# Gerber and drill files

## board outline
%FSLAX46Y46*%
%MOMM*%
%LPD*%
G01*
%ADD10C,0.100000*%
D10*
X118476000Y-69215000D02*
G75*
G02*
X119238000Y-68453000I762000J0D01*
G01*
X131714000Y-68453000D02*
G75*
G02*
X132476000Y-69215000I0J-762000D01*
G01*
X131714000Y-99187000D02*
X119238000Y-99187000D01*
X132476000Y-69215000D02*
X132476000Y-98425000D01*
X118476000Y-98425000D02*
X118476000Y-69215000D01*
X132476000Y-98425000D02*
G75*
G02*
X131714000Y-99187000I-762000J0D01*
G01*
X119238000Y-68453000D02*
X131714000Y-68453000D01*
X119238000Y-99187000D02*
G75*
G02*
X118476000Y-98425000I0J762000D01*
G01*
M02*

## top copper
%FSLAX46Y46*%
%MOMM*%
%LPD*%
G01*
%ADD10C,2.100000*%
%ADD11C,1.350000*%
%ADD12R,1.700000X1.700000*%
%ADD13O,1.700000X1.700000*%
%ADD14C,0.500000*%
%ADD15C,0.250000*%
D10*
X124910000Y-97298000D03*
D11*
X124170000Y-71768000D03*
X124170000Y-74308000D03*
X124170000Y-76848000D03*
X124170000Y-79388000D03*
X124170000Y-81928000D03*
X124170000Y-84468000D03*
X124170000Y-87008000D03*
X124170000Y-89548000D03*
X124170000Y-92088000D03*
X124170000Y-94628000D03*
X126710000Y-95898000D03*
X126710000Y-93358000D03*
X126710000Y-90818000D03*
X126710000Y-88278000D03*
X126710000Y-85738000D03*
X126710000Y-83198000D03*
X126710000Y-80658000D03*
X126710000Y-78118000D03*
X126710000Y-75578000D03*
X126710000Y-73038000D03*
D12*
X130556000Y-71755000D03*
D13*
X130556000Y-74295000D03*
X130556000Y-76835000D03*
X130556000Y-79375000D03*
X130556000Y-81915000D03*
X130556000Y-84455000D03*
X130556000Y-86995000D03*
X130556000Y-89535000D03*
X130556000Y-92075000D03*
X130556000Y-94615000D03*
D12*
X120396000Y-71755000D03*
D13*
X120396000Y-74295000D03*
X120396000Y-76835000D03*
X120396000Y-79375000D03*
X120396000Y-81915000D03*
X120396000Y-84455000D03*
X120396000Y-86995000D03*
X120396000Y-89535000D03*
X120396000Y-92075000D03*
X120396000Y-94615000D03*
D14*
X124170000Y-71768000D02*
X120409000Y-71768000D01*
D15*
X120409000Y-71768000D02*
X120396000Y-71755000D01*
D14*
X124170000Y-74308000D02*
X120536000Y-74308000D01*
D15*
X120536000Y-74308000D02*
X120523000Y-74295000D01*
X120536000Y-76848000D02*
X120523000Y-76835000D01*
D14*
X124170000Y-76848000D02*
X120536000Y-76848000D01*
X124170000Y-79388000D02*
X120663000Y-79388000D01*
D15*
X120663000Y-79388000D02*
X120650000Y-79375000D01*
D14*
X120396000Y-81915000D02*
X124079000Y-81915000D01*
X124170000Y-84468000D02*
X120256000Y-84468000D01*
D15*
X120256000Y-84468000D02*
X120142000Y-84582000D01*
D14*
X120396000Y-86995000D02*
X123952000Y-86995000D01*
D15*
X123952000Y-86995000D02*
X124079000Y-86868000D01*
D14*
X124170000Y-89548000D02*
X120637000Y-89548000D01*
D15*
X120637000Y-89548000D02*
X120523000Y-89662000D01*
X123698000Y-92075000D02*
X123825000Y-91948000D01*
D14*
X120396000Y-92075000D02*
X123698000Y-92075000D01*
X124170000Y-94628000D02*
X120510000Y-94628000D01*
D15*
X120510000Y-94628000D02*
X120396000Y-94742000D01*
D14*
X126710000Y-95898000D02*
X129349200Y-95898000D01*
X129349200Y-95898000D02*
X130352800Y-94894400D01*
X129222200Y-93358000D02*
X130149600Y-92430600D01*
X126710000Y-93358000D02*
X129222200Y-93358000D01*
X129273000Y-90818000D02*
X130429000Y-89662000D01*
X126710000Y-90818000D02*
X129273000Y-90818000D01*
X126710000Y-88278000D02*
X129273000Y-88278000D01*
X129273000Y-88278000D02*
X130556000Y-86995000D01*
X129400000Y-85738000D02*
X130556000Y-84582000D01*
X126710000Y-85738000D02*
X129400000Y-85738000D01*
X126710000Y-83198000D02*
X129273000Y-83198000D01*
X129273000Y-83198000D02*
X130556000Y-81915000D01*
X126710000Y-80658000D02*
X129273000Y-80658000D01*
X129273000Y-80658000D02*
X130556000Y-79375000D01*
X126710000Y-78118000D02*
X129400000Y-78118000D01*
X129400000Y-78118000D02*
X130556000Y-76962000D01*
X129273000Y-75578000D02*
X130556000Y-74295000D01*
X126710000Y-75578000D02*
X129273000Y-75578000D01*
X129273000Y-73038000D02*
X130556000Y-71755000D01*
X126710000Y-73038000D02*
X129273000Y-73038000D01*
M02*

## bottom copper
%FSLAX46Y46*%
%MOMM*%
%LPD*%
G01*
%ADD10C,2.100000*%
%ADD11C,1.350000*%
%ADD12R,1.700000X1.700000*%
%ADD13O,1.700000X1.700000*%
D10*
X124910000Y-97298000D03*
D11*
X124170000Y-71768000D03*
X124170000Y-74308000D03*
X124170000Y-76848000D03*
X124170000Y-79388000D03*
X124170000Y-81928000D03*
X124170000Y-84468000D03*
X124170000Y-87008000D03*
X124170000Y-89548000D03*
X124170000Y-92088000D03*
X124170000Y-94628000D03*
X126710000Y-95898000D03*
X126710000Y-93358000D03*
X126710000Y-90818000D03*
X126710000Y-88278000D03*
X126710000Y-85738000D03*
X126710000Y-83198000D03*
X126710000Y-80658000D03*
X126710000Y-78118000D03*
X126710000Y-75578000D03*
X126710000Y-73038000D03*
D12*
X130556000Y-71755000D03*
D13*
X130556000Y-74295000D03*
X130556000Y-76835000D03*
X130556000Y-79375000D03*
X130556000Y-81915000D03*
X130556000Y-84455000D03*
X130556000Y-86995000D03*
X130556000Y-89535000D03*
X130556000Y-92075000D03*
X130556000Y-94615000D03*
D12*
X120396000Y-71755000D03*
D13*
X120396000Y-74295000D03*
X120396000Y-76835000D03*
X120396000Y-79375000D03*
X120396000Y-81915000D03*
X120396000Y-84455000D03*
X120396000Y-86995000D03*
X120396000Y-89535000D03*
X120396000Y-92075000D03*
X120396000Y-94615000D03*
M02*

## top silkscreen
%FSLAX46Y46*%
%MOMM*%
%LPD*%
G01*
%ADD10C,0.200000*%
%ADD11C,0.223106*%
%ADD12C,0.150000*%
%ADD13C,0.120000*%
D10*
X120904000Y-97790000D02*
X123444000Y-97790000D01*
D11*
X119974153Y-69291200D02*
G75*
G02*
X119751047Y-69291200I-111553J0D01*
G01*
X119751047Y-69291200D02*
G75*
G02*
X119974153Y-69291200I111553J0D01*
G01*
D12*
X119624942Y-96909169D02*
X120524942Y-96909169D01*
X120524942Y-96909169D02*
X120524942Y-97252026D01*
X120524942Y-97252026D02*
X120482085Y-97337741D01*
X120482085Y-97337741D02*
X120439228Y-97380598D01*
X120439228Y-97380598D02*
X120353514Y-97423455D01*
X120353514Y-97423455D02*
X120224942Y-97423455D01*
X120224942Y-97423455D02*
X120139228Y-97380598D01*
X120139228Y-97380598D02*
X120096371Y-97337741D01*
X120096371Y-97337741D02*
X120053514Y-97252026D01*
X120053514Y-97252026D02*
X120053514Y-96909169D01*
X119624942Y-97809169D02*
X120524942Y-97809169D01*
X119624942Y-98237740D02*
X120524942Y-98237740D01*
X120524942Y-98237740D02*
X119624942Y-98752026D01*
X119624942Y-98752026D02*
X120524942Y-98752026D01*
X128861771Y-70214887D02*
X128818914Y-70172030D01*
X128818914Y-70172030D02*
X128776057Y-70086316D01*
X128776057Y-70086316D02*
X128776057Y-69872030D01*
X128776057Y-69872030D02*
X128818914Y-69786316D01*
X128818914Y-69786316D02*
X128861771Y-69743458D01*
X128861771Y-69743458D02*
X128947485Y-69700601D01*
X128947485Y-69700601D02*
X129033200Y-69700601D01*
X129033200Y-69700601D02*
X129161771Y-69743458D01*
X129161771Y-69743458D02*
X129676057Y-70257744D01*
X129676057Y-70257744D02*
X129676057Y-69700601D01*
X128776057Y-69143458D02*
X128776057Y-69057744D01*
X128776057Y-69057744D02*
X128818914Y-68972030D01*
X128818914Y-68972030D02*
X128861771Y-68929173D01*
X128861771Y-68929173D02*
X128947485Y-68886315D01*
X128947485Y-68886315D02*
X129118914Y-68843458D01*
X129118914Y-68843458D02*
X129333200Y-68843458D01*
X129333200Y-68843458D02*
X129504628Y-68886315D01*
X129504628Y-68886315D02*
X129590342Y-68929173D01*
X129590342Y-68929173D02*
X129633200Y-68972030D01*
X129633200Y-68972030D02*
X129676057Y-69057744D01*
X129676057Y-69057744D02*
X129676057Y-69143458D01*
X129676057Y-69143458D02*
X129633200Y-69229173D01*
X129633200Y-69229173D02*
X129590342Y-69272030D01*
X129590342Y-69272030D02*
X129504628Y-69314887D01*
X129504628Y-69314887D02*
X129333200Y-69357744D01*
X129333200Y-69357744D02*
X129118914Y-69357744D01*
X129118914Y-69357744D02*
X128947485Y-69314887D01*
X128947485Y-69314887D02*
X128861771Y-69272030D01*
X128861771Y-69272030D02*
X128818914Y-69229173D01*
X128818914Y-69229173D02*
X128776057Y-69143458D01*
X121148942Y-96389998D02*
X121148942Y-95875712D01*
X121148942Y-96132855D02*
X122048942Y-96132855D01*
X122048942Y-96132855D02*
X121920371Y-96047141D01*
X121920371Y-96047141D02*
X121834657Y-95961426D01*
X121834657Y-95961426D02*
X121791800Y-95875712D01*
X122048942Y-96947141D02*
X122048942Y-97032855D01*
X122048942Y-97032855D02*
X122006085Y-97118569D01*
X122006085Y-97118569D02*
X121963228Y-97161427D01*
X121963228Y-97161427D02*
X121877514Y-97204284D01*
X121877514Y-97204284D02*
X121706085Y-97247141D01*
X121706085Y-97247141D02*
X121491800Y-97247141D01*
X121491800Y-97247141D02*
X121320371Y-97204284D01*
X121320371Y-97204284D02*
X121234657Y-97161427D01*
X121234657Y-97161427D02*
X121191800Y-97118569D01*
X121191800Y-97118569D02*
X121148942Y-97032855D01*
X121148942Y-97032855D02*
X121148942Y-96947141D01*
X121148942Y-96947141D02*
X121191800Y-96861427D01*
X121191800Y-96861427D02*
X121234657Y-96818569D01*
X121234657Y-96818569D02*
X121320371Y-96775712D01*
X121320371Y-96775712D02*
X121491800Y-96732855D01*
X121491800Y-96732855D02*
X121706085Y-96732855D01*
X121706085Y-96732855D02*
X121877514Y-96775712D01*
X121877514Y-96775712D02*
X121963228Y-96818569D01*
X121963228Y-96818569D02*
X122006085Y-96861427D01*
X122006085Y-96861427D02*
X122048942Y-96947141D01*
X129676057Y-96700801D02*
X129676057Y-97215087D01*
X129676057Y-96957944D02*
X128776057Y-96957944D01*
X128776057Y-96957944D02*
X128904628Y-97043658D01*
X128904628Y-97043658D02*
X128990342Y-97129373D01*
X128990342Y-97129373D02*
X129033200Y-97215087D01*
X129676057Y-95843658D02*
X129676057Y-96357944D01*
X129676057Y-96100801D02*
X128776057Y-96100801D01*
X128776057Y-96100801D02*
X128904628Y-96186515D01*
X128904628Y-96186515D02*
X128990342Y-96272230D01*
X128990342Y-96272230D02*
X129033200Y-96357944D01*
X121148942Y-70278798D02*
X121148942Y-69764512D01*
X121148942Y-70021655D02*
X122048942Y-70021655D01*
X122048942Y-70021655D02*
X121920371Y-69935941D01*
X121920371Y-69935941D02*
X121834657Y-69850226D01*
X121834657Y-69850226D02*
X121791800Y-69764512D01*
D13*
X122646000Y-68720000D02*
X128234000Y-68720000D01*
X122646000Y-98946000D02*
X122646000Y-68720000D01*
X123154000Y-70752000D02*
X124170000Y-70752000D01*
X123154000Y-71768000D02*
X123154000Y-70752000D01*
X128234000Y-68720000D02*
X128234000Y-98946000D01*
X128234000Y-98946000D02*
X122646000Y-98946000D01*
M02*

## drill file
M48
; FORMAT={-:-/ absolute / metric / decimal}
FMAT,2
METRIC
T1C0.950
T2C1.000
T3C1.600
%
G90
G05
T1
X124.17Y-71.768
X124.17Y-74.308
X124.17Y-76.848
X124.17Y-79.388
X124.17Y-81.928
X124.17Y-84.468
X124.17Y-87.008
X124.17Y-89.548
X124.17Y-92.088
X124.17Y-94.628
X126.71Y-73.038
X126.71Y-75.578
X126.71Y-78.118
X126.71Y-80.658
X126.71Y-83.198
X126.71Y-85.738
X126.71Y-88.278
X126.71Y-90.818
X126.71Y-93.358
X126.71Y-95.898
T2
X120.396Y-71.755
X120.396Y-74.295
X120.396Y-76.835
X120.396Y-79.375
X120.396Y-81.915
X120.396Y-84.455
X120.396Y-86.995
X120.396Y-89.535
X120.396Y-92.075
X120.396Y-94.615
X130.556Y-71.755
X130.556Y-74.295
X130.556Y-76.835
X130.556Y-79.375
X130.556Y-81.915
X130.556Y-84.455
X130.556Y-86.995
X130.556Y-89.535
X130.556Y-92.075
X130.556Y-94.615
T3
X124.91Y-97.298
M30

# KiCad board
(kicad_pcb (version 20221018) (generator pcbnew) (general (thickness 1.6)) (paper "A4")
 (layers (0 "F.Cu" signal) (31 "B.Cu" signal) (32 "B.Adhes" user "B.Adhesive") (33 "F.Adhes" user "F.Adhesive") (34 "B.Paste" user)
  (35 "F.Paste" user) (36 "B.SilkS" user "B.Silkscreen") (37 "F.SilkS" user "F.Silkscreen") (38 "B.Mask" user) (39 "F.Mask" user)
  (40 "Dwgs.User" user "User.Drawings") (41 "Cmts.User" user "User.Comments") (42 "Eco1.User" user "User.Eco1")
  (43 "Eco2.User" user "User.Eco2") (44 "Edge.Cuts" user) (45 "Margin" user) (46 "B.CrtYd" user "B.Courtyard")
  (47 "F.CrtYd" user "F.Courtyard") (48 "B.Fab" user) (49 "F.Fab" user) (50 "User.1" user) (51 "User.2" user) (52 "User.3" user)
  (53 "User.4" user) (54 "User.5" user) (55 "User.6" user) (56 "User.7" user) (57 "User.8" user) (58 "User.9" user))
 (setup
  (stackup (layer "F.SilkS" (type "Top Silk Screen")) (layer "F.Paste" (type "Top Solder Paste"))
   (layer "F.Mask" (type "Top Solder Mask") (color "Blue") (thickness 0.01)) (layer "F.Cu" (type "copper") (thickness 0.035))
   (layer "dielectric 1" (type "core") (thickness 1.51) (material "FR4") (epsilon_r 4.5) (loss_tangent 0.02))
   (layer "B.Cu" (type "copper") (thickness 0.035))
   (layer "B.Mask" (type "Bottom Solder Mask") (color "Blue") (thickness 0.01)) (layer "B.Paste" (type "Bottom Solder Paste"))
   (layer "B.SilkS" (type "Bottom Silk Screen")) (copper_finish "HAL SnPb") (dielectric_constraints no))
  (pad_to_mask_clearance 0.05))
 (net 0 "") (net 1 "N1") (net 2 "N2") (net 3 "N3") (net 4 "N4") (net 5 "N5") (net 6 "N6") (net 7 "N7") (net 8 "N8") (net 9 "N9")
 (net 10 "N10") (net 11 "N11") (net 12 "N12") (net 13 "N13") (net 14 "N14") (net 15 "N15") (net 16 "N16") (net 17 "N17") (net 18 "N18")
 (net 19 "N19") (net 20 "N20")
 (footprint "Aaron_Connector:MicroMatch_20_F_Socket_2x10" (layer "F.Cu") (at 124.17 71.768)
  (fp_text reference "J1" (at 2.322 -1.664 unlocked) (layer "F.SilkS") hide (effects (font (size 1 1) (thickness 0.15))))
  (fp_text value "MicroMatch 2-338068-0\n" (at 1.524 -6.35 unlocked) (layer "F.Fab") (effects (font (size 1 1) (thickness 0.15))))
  (fp_line (start -1.524 -3.048) (end 4.064 -3.048) (stroke (width 0.12) (type default)) (layer "F.SilkS"))
  (fp_line (start -1.524 27.178) (end -1.524 -3.048) (stroke (width 0.12) (type default)) (layer "F.SilkS"))
  (fp_line (start -1.016 -1.016) (end 0 -1.016) (stroke (width 0.12) (type default)) (layer "F.SilkS"))
  (fp_line (start -1.016 0) (end -1.016 -1.016) (stroke (width 0.12) (type default)) (layer "F.SilkS"))
  (fp_line (start 4.064 -3.048) (end 4.064 27.178) (stroke (width 0.12) (type default)) (layer "F.SilkS"))
  (fp_line (start 4.064 27.178) (end -1.524 27.178) (stroke (width 0.12) (type default)) (layer "F.SilkS"))
  (pad "" thru_hole circle (at 0.74 25.53) (size 2.1 2.1) (drill 1.6) (layers "*.Cu" "*.Mask"))
  (pad "1" thru_hole circle (at 0 0) (size 1.35 1.35) (drill 0.95) (layers "*.Cu" "*.Mask") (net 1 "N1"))
  (pad "2" thru_hole circle (at 0 2.54) (size 1.35 1.35) (drill 0.95) (layers "*.Cu" "*.Mask") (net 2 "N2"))
  (pad "3" thru_hole circle (at 0 5.08) (size 1.35 1.35) (drill 0.95) (layers "*.Cu" "*.Mask") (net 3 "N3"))
  (pad "4" thru_hole circle (at 0 7.62) (size 1.35 1.35) (drill 0.95) (layers "*.Cu" "*.Mask") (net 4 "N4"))
  (pad "5" thru_hole circle (at 0 10.16) (size 1.35 1.35) (drill 0.95) (layers "*.Cu" "*.Mask") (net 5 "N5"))
  (pad "6" thru_hole circle (at 0 12.7) (size 1.35 1.35) (drill 0.95) (layers "*.Cu" "*.Mask") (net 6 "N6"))
  (pad "7" thru_hole circle (at 0 15.24) (size 1.35 1.35) (drill 0.95) (layers "*.Cu" "*.Mask") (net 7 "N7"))
  (pad "8" thru_hole circle (at 0 17.78) (size 1.35 1.35) (drill 0.95) (layers "*.Cu" "*.Mask") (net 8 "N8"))
  (pad "9" thru_hole circle (at 0 20.32) (size 1.35 1.35) (drill 0.95) (layers "*.Cu" "*.Mask") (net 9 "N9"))
  (pad "10" thru_hole circle (at 0 22.86) (size 1.35 1.35) (drill 0.95) (layers "*.Cu" "*.Mask") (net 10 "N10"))
  (pad "11" thru_hole circle (at 2.54 24.13 90) (size 1.35 1.35) (drill 0.95) (layers "*.Cu" "*.Mask") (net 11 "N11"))
  (pad "12" thru_hole circle (at 2.54 21.59) (size 1.35 1.35) (drill 0.95) (layers "*.Cu" "*.Mask") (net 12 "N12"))
  (pad "13" thru_hole circle (at 2.54 19.05) (size 1.35 1.35) (drill 0.95) (layers "*.Cu" "*.Mask") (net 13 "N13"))
  (pad "14" thru_hole circle (at 2.54 16.51) (size 1.35 1.35) (drill 0.95) (layers "*.Cu" "*.Mask") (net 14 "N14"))
  (pad "15" thru_hole circle (at 2.54 13.97) (size 1.35 1.35) (drill 0.95) (layers "*.Cu" "*.Mask") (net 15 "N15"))
  (pad "16" thru_hole circle (at 2.54 11.43) (size 1.35 1.35) (drill 0.95) (layers "*.Cu" "*.Mask") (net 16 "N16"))
  (pad "17" thru_hole circle (at 2.54 8.89) (size 1.35 1.35) (drill 0.95) (layers "*.Cu" "*.Mask") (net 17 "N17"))
  (pad "18" thru_hole circle (at 2.54 6.35) (size 1.35 1.35) (drill 0.95) (layers "*.Cu" "*.Mask") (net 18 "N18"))
  (pad "19" thru_hole circle (at 2.54 3.81) (size 1.35 1.35) (drill 0.95) (layers "*.Cu" "*.Mask") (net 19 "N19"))
  (pad "20" thru_hole circle (at 2.54 1.27) (size 1.35 1.35) (drill 0.95) (layers "*.Cu" "*.Mask") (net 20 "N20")))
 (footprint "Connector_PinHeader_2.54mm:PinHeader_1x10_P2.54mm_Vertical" (layer "B.Cu") (at 130.556 71.755 180)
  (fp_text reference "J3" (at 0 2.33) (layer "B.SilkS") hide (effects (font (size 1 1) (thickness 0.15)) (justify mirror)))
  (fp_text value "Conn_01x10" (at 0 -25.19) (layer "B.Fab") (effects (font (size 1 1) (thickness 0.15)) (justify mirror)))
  (pad "1" thru_hole rect (at 0 0 180) (size 1.7 1.7) (drill 1) (layers "*.Cu" "*.Mask") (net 20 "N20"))
  (pad "2" thru_hole oval (at 0 -2.54 180) (size 1.7 1.7) (drill 1) (layers "*.Cu" "*.Mask") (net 19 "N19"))
  (pad "3" thru_hole oval (at 0 -5.08 180) (size 1.7 1.7) (drill 1) (layers "*.Cu" "*.Mask") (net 18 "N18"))
  (pad "4" thru_hole oval (at 0 -7.62 180) (size 1.7 1.7) (drill 1) (layers "*.Cu" "*.Mask") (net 17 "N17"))
  (pad "5" thru_hole oval (at 0 -10.16 180) (size 1.7 1.7) (drill 1) (layers "*.Cu" "*.Mask") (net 16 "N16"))
  (pad "6" thru_hole oval (at 0 -12.7 180) (size 1.7 1.7) (drill 1) (layers "*.Cu" "*.Mask") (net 15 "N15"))
  (pad "7" thru_hole oval (at 0 -15.24 180) (size 1.7 1.7) (drill 1) (layers "*.Cu" "*.Mask") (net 14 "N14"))
  (pad "8" thru_hole oval (at 0 -17.78 180) (size 1.7 1.7) (drill 1) (layers "*.Cu" "*.Mask") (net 13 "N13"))
  (pad "9" thru_hole oval (at 0 -20.32 180) (size 1.7 1.7) (drill 1) (layers "*.Cu" "*.Mask") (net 12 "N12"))
  (pad "10" thru_hole oval (at 0 -22.86 180) (size 1.7 1.7) (drill 1) (layers "*.Cu" "*.Mask") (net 11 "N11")))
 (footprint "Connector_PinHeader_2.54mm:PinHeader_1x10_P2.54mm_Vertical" (layer "B.Cu") (at 120.396 71.755 180)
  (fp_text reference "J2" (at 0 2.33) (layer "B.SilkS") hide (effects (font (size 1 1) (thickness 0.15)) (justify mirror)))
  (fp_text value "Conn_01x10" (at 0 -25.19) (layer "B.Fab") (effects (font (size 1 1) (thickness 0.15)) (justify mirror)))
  (pad "1" thru_hole rect (at 0 0 180) (size 1.7 1.7) (drill 1) (layers "*.Cu" "*.Mask") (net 1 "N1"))
  (pad "2" thru_hole oval (at 0 -2.54 180) (size 1.7 1.7) (drill 1) (layers "*.Cu" "*.Mask") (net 2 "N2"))
  (pad "3" thru_hole oval (at 0 -5.08 180) (size 1.7 1.7) (drill 1) (layers "*.Cu" "*.Mask") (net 3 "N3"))
  (pad "4" thru_hole oval (at 0 -7.62 180) (size 1.7 1.7) (drill 1) (layers "*.Cu" "*.Mask") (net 4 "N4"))
  (pad "5" thru_hole oval (at 0 -10.16 180) (size 1.7 1.7) (drill 1) (layers "*.Cu" "*.Mask") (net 5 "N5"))
  (pad "6" thru_hole oval (at 0 -12.7 180) (size 1.7 1.7) (drill 1) (layers "*.Cu" "*.Mask") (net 6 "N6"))
  (pad "7" thru_hole oval (at 0 -15.24 180) (size 1.7 1.7) (drill 1) (layers "*.Cu" "*.Mask") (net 7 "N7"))
  (pad "8" thru_hole oval (at 0 -17.78 180) (size 1.7 1.7) (drill 1) (layers "*.Cu" "*.Mask") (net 8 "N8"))
  (pad "9" thru_hole oval (at 0 -20.32 180) (size 1.7 1.7) (drill 1) (layers "*.Cu" "*.Mask") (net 9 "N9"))
  (pad "10" thru_hole oval (at 0 -22.86 180) (size 1.7 1.7) (drill 1) (layers "*.Cu" "*.Mask") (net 10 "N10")))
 (gr_line (start 120.904 97.79) (end 123.444 97.79) (stroke (width 0.2) (type default)) (layer "F.SilkS"))
 (gr_circle (center 119.8626 69.2912) (end 120.010706 69.2912) (stroke (width 0.15) (type solid)) (fill solid) (layer "F.SilkS"))
 (gr_arc (start 118.476 69.215) (mid 118.699185 68.676185) (end 119.238 68.453) (stroke (width 0.1) (type default)) (layer "Edge.Cuts"))
 (gr_arc (start 131.714 68.453) (mid 132.252815 68.676185) (end 132.476 69.215) (stroke (width 0.1) (type default)) (layer "Edge.Cuts"))
 (gr_line (start 131.714 99.187) (end 119.238 99.187) (stroke (width 0.1) (type default)) (layer "Edge.Cuts"))
 (gr_line (start 132.476 69.215) (end 132.476 98.425) (stroke (width 0.1) (type default)) (layer "Edge.Cuts"))
 (gr_line (start 118.476 98.425) (end 118.476 69.215) (stroke (width 0.1) (type default)) (layer "Edge.Cuts"))
 (gr_arc (start 132.476 98.425) (mid 132.252815 98.963815) (end 131.714 99.187) (stroke (width 0.1) (type default)) (layer "Edge.Cuts"))
 (gr_line (start 119.238 68.453) (end 131.714 68.453) (stroke (width 0.1) (type default)) (layer "Edge.Cuts"))
 (gr_arc (start 119.238 99.187) (mid 118.699185 98.963815) (end 118.476 98.425) (stroke (width 0.1) (type default)) (layer "Edge.Cuts"))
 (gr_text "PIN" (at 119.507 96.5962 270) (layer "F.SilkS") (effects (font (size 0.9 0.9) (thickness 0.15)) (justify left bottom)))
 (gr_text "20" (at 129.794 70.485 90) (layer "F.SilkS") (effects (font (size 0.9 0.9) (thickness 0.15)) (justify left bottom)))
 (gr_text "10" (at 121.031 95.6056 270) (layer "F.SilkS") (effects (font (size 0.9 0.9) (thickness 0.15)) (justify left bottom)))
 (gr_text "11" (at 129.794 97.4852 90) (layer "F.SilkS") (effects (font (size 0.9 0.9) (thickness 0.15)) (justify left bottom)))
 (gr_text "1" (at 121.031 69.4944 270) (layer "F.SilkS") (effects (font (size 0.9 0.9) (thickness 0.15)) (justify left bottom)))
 (segment (start 124.17 71.768) (end 120.409 71.768) (width 0.5) (layer "F.Cu") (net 1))
 (segment (start 120.409 71.768) (end 120.396 71.755) (width 0.25) (layer "F.Cu") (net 1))
 (segment (start 124.17 74.308) (end 120.536 74.308) (width 0.5) (layer "F.Cu") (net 2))
 (segment (start 120.536 74.308) (end 120.523 74.295) (width 0.25) (layer "F.Cu") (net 2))
 (segment (start 120.536 76.848) (end 120.523 76.835) (width 0.25) (layer "F.Cu") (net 3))
 (segment (start 124.17 76.848) (end 120.536 76.848) (width 0.5) (layer "F.Cu") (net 3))
 (segment (start 124.17 79.388) (end 120.663 79.388) (width 0.5) (layer "F.Cu") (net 4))
 (segment (start 120.663 79.388) (end 120.65 79.375) (width 0.25) (layer "F.Cu") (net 4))
 (segment (start 120.396 81.915) (end 124.079 81.915) (width 0.5) (layer "F.Cu") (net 5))
 (segment (start 124.17 84.468) (end 120.256 84.468) (width 0.5) (layer "F.Cu") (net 6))
 (segment (start 120.256 84.468) (end 120.142 84.582) (width 0.25) (layer "F.Cu") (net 6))
 (segment (start 120.396 86.995) (end 123.952 86.995) (width 0.5) (layer "F.Cu") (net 7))
 (segment (start 123.952 86.995) (end 124.079 86.868) (width 0.25) (layer "F.Cu") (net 7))
 (segment (start 124.17 89.548) (end 120.637 89.548) (width 0.5) (layer "F.Cu") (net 8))
 (segment (start 120.637 89.548) (end 120.523 89.662) (width 0.25) (layer "F.Cu") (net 8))
 (segment (start 123.698 92.075) (end 123.825 91.948) (width 0.25) (layer "F.Cu") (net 9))
 (segment (start 120.396 92.075) (end 123.698 92.075) (width 0.5) (layer "F.Cu") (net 9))
 (segment (start 124.17 94.628) (end 120.51 94.628) (width 0.5) (layer "F.Cu") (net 10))
 (segment (start 120.51 94.628) (end 120.396 94.742) (width 0.25) (layer "F.Cu") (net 10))
 (segment (start 126.71 95.898) (end 129.3492 95.898) (width 0.5) (layer "F.Cu") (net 11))
 (segment (start 129.3492 95.898) (end 130.3528 94.8944) (width 0.5) (layer "F.Cu") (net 11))
 (segment (start 129.2222 93.358) (end 130.1496 92.4306) (width 0.5) (layer "F.Cu") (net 12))
 (segment (start 126.71 93.358) (end 129.2222 93.358) (width 0.5) (layer "F.Cu") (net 12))
 (segment (start 129.273 90.818) (end 130.429 89.662) (width 0.5) (layer "F.Cu") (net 13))
 (segment (start 126.71 90.818) (end 129.273 90.818) (width 0.5) (layer "F.Cu") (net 13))
 (segment (start 126.71 88.278) (end 129.273 88.278) (width 0.5) (layer "F.Cu") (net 14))
 (segment (start 129.273 88.278) (end 130.556 86.995) (width 0.5) (layer "F.Cu") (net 14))
 (segment (start 129.4 85.738) (end 130.556 84.582) (width 0.5) (layer "F.Cu") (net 15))
 (segment (start 126.71 85.738) (end 129.4 85.738) (width 0.5) (layer "F.Cu") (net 15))
 (segment (start 126.71 83.198) (end 129.273 83.198) (width 0.5) (layer "F.Cu") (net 16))
 (segment (start 129.273 83.198) (end 130.556 81.915) (width 0.5) (layer "F.Cu") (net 16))
 (segment (start 126.71 80.658) (end 129.273 80.658) (width 0.5) (layer "F.Cu") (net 17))
 (segment (start 129.273 80.658) (end 130.556 79.375) (width 0.5) (layer "F.Cu") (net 17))
 (segment (start 126.71 78.118) (end 129.4 78.118) (width 0.5) (layer "F.Cu") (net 18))
 (segment (start 129.4 78.118) (end 130.556 76.962) (width 0.5) (layer "F.Cu") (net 18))
 (segment (start 129.273 75.578) (end 130.556 74.295) (width 0.5) (layer "F.Cu") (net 19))
 (segment (start 126.71 75.578) (end 129.273 75.578) (width 0.5) (layer "F.Cu") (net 19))
 (segment (start 129.273 73.038) (end 130.556 71.755) (width 0.5) (layer "F.Cu") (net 20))
 (segment (start 126.71 73.038) (end 129.273 73.038) (width 0.5) (layer "F.Cu") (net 20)))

